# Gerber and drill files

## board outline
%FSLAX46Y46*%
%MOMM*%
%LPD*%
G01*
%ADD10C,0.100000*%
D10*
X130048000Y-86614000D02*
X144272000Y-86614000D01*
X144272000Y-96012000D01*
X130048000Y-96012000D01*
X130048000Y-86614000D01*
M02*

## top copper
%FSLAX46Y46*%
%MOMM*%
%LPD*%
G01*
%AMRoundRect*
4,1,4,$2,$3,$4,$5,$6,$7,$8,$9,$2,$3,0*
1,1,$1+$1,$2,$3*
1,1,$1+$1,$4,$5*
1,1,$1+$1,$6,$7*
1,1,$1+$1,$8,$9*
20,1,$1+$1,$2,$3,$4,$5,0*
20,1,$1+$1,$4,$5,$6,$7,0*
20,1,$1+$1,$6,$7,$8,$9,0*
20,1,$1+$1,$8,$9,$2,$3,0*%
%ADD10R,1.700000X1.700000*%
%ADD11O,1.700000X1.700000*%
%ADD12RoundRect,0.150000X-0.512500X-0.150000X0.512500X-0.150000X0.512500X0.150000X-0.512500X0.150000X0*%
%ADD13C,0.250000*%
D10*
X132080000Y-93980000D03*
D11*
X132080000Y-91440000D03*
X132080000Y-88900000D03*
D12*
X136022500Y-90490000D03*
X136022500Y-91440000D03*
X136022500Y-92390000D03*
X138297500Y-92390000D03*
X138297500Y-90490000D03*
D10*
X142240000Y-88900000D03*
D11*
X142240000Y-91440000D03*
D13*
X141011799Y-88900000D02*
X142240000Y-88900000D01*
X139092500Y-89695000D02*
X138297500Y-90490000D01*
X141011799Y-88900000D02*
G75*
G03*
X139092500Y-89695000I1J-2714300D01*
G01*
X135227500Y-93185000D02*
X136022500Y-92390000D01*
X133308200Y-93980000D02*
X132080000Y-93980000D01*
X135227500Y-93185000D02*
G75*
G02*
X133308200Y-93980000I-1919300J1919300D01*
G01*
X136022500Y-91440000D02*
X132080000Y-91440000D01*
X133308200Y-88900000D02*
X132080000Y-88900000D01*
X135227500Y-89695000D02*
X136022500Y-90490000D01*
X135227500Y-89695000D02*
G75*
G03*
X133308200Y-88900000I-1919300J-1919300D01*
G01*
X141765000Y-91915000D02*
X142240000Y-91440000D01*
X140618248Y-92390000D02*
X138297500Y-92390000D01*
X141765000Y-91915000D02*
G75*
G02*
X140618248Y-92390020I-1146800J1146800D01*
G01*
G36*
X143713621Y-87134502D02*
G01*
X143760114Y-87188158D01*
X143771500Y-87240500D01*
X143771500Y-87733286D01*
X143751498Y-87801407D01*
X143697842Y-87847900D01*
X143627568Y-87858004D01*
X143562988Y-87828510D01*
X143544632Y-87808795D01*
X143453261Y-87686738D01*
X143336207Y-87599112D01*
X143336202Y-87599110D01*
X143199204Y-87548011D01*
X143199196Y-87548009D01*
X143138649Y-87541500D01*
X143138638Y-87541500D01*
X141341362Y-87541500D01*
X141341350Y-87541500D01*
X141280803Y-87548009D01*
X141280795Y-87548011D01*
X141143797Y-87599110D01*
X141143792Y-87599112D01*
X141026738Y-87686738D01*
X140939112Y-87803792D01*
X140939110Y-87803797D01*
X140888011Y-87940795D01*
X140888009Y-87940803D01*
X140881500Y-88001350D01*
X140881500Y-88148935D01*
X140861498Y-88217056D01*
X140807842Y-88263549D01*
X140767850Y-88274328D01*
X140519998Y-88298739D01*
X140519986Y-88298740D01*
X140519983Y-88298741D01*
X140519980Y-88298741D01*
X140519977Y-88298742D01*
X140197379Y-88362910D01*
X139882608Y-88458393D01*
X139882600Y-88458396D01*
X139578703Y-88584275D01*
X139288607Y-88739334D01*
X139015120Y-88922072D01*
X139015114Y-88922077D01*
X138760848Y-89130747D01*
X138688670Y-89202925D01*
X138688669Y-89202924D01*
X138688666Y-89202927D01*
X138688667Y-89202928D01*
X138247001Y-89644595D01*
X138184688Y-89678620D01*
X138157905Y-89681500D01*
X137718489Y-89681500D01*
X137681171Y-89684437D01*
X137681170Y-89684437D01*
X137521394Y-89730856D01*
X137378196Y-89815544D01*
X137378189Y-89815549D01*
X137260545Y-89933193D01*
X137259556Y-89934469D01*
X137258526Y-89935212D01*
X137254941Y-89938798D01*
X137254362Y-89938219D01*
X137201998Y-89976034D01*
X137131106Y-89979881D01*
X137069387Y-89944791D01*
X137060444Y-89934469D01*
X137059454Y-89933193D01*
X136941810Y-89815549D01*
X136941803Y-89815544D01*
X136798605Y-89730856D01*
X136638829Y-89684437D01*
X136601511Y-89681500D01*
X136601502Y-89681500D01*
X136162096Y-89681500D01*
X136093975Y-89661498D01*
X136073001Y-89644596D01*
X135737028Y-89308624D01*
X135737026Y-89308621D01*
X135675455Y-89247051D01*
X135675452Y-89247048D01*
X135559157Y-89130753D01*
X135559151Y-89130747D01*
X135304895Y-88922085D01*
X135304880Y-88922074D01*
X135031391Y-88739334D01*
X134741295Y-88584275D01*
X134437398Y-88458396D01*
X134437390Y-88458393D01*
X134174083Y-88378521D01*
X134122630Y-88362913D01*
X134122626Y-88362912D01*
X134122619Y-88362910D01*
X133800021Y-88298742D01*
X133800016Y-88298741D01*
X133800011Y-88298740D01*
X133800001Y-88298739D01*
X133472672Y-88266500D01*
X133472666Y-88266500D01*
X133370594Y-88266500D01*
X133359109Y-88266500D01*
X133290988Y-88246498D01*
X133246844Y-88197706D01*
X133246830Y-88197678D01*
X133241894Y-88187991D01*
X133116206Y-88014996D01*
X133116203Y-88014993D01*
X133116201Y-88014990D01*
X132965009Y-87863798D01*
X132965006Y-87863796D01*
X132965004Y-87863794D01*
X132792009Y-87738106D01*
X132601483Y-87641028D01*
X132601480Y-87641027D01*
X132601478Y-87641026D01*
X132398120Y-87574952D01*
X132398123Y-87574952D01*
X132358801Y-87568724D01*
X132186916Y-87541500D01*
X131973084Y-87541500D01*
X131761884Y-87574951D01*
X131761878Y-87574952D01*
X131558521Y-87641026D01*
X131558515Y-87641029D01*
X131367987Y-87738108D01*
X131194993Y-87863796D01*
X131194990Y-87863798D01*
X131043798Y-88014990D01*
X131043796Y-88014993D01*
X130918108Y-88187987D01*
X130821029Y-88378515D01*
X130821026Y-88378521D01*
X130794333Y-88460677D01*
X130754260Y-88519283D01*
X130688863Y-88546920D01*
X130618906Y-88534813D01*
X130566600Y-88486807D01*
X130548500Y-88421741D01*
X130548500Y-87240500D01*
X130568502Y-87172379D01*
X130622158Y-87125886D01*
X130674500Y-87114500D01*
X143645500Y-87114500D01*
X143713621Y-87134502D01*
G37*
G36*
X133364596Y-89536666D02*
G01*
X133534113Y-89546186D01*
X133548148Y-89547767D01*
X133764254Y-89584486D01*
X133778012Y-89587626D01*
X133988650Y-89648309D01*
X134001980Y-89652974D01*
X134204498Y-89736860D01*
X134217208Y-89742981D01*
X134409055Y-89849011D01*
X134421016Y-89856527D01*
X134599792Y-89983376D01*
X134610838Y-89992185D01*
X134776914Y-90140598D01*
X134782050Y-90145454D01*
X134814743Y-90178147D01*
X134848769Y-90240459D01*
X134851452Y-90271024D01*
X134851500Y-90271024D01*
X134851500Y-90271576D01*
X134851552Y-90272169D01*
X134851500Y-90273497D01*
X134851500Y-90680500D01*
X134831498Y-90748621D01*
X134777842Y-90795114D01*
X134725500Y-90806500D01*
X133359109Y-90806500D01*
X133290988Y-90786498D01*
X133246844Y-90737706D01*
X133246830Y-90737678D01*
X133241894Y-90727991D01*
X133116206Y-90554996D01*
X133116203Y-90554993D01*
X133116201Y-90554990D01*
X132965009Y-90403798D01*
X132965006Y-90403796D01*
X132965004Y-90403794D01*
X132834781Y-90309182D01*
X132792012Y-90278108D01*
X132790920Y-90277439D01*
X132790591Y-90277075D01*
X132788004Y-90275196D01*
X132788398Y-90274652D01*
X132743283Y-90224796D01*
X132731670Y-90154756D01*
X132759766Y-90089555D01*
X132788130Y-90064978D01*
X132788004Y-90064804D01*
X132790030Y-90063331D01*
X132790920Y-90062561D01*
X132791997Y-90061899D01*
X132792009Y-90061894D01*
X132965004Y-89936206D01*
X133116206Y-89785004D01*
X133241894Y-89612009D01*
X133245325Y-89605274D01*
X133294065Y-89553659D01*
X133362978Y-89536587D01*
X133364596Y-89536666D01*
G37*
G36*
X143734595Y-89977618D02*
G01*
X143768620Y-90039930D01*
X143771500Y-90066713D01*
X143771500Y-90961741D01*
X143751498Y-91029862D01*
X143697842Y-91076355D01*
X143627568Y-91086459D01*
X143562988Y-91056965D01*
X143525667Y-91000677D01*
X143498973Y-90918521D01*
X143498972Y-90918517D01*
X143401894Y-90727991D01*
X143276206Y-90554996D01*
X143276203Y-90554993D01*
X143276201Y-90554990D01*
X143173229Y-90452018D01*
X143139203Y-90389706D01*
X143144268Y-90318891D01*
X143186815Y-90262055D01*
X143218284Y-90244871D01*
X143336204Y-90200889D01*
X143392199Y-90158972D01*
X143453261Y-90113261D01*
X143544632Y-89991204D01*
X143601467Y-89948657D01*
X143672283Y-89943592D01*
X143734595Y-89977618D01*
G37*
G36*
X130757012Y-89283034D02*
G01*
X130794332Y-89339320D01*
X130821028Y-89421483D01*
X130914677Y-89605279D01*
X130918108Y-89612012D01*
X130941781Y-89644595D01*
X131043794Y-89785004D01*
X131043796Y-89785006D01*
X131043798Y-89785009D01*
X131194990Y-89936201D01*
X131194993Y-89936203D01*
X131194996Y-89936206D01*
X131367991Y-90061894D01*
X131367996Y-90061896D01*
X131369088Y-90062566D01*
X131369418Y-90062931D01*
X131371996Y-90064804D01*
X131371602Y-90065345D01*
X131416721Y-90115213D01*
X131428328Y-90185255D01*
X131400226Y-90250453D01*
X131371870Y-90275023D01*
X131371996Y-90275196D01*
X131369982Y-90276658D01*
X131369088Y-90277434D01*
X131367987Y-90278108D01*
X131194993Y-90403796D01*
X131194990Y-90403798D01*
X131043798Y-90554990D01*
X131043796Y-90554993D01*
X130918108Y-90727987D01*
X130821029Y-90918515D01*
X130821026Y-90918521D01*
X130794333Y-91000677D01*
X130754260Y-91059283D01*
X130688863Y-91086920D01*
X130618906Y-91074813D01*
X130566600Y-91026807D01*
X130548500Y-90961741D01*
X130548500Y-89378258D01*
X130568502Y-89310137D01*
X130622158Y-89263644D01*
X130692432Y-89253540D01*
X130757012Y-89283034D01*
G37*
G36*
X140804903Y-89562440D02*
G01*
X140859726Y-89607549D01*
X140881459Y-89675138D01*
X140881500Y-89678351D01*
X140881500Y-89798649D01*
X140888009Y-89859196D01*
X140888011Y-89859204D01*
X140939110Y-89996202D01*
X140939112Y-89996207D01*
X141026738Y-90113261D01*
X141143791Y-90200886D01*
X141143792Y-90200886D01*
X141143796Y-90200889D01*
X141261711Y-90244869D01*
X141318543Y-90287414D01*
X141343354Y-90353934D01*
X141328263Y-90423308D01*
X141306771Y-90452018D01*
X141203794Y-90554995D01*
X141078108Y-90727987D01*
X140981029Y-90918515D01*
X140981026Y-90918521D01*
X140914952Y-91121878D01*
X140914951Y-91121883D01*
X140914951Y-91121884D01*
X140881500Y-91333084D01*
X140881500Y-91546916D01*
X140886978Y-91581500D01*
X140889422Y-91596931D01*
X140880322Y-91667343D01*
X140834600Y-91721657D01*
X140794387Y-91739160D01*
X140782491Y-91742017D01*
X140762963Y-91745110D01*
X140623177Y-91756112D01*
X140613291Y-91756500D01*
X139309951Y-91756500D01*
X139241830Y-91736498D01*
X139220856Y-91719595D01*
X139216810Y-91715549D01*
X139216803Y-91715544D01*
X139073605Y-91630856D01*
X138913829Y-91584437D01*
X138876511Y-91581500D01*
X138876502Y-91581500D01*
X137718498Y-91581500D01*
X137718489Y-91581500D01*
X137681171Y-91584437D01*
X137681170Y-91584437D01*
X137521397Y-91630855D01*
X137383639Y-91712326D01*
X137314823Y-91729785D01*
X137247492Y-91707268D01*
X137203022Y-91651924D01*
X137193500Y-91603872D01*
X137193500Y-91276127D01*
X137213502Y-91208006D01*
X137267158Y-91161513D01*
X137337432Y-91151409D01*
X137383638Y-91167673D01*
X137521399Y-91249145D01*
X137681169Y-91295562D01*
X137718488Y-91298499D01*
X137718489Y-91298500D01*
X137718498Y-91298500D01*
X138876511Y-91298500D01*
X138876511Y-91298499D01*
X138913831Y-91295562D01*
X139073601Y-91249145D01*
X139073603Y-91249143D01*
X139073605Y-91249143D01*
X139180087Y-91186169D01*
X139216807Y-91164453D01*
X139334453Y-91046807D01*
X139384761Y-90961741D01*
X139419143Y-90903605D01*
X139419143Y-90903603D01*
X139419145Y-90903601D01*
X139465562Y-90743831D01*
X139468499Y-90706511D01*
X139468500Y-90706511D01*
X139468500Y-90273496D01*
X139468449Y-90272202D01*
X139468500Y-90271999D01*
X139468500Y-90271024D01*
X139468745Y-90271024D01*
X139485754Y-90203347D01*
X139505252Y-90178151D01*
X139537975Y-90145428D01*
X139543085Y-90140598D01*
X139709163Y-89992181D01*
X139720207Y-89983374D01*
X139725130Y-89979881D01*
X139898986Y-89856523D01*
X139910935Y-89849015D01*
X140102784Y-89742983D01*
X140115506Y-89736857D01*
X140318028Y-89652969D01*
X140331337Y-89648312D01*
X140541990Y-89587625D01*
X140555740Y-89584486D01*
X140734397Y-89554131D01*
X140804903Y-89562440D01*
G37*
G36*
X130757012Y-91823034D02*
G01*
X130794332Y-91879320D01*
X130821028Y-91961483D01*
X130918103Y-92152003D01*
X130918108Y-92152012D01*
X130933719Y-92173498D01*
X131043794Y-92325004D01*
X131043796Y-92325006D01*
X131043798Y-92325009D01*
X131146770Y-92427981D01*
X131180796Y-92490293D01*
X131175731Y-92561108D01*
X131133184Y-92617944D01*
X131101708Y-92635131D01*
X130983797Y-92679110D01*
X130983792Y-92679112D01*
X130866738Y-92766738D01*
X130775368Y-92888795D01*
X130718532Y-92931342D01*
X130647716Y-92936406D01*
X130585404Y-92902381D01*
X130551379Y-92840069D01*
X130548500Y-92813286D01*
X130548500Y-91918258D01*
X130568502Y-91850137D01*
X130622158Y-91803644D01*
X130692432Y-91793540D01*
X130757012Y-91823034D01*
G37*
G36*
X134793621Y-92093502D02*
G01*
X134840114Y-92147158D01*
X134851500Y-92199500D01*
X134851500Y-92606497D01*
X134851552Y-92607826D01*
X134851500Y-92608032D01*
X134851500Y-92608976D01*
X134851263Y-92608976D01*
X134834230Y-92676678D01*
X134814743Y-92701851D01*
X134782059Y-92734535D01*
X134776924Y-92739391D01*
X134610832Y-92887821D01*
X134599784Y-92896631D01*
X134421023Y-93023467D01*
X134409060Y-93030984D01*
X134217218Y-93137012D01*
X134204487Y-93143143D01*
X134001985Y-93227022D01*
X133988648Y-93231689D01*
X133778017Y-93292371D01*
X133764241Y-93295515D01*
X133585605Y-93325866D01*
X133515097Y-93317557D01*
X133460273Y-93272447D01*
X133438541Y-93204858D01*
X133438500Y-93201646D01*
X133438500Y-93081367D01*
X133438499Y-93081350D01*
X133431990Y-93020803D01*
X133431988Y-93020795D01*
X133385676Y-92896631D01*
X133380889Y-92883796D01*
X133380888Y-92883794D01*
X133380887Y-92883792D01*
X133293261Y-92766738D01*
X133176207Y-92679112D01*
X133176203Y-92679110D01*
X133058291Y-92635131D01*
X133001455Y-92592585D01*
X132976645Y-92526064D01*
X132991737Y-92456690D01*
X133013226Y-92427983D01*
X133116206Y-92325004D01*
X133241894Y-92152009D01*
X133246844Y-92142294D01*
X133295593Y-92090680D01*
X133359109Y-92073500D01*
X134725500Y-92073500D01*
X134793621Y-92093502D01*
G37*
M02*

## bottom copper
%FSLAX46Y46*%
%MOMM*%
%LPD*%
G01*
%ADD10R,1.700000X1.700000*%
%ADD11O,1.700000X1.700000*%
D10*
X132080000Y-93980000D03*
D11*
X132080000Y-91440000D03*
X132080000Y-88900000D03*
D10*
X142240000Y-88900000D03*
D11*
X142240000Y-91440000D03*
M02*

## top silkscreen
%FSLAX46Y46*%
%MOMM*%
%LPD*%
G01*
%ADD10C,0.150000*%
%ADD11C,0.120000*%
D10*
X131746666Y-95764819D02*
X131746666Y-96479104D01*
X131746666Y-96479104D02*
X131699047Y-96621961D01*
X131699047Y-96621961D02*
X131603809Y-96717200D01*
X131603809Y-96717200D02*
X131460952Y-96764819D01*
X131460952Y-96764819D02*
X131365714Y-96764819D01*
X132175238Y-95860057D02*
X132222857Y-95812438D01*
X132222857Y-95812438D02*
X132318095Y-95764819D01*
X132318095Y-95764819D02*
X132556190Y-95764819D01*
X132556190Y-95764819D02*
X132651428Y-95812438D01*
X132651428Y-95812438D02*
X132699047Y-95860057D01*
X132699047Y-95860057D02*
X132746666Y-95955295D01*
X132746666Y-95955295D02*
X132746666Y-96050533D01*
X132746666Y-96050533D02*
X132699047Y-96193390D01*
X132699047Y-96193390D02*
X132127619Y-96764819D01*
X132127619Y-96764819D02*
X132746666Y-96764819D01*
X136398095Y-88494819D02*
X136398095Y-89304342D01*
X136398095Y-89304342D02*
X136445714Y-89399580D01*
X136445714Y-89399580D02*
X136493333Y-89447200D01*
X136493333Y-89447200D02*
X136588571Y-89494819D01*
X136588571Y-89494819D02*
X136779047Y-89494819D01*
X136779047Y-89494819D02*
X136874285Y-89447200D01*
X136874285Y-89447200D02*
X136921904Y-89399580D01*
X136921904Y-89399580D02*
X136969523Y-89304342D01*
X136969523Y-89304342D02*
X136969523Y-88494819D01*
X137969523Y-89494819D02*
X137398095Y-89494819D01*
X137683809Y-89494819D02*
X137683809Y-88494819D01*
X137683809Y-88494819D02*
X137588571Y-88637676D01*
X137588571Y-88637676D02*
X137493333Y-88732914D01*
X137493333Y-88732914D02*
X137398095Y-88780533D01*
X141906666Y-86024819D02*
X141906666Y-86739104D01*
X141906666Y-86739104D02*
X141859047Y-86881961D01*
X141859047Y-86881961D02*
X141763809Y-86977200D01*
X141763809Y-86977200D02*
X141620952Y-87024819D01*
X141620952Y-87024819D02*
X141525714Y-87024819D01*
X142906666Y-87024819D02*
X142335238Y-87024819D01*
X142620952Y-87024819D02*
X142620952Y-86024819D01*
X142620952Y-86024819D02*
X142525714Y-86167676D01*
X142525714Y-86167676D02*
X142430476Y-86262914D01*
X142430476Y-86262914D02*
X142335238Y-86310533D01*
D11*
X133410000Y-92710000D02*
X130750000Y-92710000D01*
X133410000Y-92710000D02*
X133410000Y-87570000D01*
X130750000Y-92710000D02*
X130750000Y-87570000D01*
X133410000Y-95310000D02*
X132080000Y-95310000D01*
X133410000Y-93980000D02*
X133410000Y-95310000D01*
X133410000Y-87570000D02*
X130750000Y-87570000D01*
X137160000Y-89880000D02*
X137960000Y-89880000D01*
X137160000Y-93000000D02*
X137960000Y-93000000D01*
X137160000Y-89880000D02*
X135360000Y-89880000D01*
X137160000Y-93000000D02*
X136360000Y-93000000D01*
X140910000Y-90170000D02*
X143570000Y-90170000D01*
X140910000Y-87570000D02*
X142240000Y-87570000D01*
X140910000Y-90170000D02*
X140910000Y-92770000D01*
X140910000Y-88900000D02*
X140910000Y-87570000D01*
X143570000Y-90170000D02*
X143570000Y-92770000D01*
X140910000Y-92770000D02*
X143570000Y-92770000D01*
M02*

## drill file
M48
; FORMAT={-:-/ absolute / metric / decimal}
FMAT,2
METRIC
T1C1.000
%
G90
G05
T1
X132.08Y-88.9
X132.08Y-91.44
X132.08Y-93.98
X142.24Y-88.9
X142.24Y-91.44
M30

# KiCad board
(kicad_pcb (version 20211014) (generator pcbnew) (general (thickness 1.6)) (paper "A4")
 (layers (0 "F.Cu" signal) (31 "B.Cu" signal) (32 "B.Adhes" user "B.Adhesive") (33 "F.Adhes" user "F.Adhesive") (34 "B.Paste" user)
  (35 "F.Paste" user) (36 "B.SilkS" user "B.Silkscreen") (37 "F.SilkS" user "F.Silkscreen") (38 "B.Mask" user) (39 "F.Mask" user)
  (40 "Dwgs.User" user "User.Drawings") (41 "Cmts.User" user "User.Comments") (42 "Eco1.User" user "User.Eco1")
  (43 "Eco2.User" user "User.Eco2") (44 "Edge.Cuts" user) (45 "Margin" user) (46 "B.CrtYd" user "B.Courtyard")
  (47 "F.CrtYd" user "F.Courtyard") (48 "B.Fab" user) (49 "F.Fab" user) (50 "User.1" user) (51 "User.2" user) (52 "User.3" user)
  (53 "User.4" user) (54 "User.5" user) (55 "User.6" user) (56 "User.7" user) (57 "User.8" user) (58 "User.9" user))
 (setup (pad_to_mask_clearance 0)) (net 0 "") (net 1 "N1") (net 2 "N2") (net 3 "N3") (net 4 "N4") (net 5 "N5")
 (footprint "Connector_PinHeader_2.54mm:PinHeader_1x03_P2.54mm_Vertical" (layer "F.Cu") (at 132.08 93.98 180)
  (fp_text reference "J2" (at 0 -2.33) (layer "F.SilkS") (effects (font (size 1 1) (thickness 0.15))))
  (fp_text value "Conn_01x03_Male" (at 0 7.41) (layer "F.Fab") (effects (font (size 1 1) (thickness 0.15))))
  (fp_line (start -1.33 1.27) (end 1.33 1.27) (layer "F.SilkS") (width 0.12))
  (fp_line (start -1.33 1.27) (end -1.33 6.41) (layer "F.SilkS") (width 0.12))
  (fp_line (start 1.33 1.27) (end 1.33 6.41) (layer "F.SilkS") (width 0.12))
  (fp_line (start -1.33 -1.33) (end 0 -1.33) (layer "F.SilkS") (width 0.12))
  (fp_line (start -1.33 0) (end -1.33 -1.33) (layer "F.SilkS") (width 0.12))
  (fp_line (start -1.33 6.41) (end 1.33 6.41) (layer "F.SilkS") (width 0.12))
  (pad "1" thru_hole rect (at 0 0 180) (size 1.7 1.7) (drill 1) (layers *.Cu *.Mask) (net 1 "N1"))
  (pad "2" thru_hole oval (at 0 2.54 180) (size 1.7 1.7) (drill 1) (layers *.Cu *.Mask) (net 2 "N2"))
  (pad "3" thru_hole oval (at 0 5.08 180) (size 1.7 1.7) (drill 1) (layers *.Cu *.Mask) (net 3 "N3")))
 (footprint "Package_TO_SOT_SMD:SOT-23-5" (layer "F.Cu") (at 137.16 91.44)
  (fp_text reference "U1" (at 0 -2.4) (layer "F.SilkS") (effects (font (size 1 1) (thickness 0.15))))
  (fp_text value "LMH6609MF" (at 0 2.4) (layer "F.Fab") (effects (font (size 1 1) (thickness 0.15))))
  (fp_line (start 0 -1.56) (end 0.8 -1.56) (layer "F.SilkS") (width 0.12))
  (fp_line (start 0 1.56) (end 0.8 1.56) (layer "F.SilkS") (width 0.12))
  (fp_line (start 0 -1.56) (end -1.8 -1.56) (layer "F.SilkS") (width 0.12))
  (fp_line (start 0 1.56) (end -0.8 1.56) (layer "F.SilkS") (width 0.12))
  (pad "1" smd roundrect (at -1.1375 -0.95) (size 1.325 0.6) (layers "F.Cu" "F.Paste" "F.Mask") (roundrect_rratio 0.25) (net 3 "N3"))
  (pad "2" smd roundrect (at -1.1375 0) (size 1.325 0.6) (layers "F.Cu" "F.Paste" "F.Mask") (roundrect_rratio 0.25) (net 2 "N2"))
  (pad "3" smd roundrect (at -1.1375 0.95) (size 1.325 0.6) (layers "F.Cu" "F.Paste" "F.Mask") (roundrect_rratio 0.25) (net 1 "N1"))
  (pad "4" smd roundrect (at 1.1375 0.95) (size 1.325 0.6) (layers "F.Cu" "F.Paste" "F.Mask") (roundrect_rratio 0.25) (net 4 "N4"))
  (pad "5" smd roundrect (at 1.1375 -0.95) (size 1.325 0.6) (layers "F.Cu" "F.Paste" "F.Mask") (roundrect_rratio 0.25) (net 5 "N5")))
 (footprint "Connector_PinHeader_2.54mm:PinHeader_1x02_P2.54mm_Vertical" (layer "F.Cu") (at 142.24 88.9)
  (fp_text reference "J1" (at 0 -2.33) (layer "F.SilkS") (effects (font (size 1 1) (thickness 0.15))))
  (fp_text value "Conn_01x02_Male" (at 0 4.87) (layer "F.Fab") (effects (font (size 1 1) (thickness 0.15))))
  (fp_line (start -1.33 1.27) (end 1.33 1.27) (layer "F.SilkS") (width 0.12))
  (fp_line (start -1.33 -1.33) (end 0 -1.33) (layer "F.SilkS") (width 0.12))
  (fp_line (start -1.33 1.27) (end -1.33 3.87) (layer "F.SilkS") (width 0.12))
  (fp_line (start -1.33 0) (end -1.33 -1.33) (layer "F.SilkS") (width 0.12))
  (fp_line (start 1.33 1.27) (end 1.33 3.87) (layer "F.SilkS") (width 0.12))
  (fp_line (start -1.33 3.87) (end 1.33 3.87) (layer "F.SilkS") (width 0.12))
  (pad "1" thru_hole rect (at 0 0) (size 1.7 1.7) (drill 1) (layers *.Cu *.Mask) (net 5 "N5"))
  (pad "2" thru_hole oval (at 0 2.54) (size 1.7 1.7) (drill 1) (layers *.Cu *.Mask) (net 4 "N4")))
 (gr_rect (start 130.048 86.614) (end 144.272 96.012) (layer "Edge.Cuts") (width 0.1) (fill none))
 (segment (start 141.011799 88.9) (end 142.24 88.9) (width 0.25) (layer "F.Cu") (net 5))
 (segment (start 139.0925 89.695) (end 138.2975 90.49) (width 0.25) (layer "F.Cu") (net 5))
 (arc (start 141.011799 88.9) (mid 139.973082 89.106613) (end 139.0925 89.695) (width 0.25) (layer "F.Cu") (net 5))
 (segment (start 135.2275 93.185) (end 136.0225 92.39) (width 0.25) (layer "F.Cu") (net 1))
 (segment (start 133.3082 93.98) (end 132.08 93.98) (width 0.25) (layer "F.Cu") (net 1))
 (arc (start 135.2275 93.185) (mid 134.346917 93.773386) (end 133.3082 93.98) (width 0.25) (layer "F.Cu") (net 1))
 (segment (start 136.0225 91.44) (end 132.08 91.44) (width 0.25) (layer "F.Cu") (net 2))
 (segment (start 133.3082 88.9) (end 132.08 88.9) (width 0.25) (layer "F.Cu") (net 3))
 (segment (start 135.2275 89.695) (end 136.0225 90.49) (width 0.25) (layer "F.Cu") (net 3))
 (arc (start 135.2275 89.695) (mid 134.346917 89.106613) (end 133.3082 88.9) (width 0.25) (layer "F.Cu") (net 3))
 (segment (start 141.765 91.915) (end 142.24 91.44) (width 0.25) (layer "F.Cu") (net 4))
 (segment (start 140.618248 92.39) (end 138.2975 92.39) (width 0.25) (layer "F.Cu") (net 4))
 (arc (start 141.765 91.915) (mid 141.238865 92.266551) (end 140.618248 92.39) (width 0.25) (layer "F.Cu") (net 4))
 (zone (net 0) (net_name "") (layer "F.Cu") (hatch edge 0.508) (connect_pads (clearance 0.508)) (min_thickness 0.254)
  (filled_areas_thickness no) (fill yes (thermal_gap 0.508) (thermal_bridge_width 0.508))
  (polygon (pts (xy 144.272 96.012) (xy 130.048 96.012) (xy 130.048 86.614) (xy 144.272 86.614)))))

